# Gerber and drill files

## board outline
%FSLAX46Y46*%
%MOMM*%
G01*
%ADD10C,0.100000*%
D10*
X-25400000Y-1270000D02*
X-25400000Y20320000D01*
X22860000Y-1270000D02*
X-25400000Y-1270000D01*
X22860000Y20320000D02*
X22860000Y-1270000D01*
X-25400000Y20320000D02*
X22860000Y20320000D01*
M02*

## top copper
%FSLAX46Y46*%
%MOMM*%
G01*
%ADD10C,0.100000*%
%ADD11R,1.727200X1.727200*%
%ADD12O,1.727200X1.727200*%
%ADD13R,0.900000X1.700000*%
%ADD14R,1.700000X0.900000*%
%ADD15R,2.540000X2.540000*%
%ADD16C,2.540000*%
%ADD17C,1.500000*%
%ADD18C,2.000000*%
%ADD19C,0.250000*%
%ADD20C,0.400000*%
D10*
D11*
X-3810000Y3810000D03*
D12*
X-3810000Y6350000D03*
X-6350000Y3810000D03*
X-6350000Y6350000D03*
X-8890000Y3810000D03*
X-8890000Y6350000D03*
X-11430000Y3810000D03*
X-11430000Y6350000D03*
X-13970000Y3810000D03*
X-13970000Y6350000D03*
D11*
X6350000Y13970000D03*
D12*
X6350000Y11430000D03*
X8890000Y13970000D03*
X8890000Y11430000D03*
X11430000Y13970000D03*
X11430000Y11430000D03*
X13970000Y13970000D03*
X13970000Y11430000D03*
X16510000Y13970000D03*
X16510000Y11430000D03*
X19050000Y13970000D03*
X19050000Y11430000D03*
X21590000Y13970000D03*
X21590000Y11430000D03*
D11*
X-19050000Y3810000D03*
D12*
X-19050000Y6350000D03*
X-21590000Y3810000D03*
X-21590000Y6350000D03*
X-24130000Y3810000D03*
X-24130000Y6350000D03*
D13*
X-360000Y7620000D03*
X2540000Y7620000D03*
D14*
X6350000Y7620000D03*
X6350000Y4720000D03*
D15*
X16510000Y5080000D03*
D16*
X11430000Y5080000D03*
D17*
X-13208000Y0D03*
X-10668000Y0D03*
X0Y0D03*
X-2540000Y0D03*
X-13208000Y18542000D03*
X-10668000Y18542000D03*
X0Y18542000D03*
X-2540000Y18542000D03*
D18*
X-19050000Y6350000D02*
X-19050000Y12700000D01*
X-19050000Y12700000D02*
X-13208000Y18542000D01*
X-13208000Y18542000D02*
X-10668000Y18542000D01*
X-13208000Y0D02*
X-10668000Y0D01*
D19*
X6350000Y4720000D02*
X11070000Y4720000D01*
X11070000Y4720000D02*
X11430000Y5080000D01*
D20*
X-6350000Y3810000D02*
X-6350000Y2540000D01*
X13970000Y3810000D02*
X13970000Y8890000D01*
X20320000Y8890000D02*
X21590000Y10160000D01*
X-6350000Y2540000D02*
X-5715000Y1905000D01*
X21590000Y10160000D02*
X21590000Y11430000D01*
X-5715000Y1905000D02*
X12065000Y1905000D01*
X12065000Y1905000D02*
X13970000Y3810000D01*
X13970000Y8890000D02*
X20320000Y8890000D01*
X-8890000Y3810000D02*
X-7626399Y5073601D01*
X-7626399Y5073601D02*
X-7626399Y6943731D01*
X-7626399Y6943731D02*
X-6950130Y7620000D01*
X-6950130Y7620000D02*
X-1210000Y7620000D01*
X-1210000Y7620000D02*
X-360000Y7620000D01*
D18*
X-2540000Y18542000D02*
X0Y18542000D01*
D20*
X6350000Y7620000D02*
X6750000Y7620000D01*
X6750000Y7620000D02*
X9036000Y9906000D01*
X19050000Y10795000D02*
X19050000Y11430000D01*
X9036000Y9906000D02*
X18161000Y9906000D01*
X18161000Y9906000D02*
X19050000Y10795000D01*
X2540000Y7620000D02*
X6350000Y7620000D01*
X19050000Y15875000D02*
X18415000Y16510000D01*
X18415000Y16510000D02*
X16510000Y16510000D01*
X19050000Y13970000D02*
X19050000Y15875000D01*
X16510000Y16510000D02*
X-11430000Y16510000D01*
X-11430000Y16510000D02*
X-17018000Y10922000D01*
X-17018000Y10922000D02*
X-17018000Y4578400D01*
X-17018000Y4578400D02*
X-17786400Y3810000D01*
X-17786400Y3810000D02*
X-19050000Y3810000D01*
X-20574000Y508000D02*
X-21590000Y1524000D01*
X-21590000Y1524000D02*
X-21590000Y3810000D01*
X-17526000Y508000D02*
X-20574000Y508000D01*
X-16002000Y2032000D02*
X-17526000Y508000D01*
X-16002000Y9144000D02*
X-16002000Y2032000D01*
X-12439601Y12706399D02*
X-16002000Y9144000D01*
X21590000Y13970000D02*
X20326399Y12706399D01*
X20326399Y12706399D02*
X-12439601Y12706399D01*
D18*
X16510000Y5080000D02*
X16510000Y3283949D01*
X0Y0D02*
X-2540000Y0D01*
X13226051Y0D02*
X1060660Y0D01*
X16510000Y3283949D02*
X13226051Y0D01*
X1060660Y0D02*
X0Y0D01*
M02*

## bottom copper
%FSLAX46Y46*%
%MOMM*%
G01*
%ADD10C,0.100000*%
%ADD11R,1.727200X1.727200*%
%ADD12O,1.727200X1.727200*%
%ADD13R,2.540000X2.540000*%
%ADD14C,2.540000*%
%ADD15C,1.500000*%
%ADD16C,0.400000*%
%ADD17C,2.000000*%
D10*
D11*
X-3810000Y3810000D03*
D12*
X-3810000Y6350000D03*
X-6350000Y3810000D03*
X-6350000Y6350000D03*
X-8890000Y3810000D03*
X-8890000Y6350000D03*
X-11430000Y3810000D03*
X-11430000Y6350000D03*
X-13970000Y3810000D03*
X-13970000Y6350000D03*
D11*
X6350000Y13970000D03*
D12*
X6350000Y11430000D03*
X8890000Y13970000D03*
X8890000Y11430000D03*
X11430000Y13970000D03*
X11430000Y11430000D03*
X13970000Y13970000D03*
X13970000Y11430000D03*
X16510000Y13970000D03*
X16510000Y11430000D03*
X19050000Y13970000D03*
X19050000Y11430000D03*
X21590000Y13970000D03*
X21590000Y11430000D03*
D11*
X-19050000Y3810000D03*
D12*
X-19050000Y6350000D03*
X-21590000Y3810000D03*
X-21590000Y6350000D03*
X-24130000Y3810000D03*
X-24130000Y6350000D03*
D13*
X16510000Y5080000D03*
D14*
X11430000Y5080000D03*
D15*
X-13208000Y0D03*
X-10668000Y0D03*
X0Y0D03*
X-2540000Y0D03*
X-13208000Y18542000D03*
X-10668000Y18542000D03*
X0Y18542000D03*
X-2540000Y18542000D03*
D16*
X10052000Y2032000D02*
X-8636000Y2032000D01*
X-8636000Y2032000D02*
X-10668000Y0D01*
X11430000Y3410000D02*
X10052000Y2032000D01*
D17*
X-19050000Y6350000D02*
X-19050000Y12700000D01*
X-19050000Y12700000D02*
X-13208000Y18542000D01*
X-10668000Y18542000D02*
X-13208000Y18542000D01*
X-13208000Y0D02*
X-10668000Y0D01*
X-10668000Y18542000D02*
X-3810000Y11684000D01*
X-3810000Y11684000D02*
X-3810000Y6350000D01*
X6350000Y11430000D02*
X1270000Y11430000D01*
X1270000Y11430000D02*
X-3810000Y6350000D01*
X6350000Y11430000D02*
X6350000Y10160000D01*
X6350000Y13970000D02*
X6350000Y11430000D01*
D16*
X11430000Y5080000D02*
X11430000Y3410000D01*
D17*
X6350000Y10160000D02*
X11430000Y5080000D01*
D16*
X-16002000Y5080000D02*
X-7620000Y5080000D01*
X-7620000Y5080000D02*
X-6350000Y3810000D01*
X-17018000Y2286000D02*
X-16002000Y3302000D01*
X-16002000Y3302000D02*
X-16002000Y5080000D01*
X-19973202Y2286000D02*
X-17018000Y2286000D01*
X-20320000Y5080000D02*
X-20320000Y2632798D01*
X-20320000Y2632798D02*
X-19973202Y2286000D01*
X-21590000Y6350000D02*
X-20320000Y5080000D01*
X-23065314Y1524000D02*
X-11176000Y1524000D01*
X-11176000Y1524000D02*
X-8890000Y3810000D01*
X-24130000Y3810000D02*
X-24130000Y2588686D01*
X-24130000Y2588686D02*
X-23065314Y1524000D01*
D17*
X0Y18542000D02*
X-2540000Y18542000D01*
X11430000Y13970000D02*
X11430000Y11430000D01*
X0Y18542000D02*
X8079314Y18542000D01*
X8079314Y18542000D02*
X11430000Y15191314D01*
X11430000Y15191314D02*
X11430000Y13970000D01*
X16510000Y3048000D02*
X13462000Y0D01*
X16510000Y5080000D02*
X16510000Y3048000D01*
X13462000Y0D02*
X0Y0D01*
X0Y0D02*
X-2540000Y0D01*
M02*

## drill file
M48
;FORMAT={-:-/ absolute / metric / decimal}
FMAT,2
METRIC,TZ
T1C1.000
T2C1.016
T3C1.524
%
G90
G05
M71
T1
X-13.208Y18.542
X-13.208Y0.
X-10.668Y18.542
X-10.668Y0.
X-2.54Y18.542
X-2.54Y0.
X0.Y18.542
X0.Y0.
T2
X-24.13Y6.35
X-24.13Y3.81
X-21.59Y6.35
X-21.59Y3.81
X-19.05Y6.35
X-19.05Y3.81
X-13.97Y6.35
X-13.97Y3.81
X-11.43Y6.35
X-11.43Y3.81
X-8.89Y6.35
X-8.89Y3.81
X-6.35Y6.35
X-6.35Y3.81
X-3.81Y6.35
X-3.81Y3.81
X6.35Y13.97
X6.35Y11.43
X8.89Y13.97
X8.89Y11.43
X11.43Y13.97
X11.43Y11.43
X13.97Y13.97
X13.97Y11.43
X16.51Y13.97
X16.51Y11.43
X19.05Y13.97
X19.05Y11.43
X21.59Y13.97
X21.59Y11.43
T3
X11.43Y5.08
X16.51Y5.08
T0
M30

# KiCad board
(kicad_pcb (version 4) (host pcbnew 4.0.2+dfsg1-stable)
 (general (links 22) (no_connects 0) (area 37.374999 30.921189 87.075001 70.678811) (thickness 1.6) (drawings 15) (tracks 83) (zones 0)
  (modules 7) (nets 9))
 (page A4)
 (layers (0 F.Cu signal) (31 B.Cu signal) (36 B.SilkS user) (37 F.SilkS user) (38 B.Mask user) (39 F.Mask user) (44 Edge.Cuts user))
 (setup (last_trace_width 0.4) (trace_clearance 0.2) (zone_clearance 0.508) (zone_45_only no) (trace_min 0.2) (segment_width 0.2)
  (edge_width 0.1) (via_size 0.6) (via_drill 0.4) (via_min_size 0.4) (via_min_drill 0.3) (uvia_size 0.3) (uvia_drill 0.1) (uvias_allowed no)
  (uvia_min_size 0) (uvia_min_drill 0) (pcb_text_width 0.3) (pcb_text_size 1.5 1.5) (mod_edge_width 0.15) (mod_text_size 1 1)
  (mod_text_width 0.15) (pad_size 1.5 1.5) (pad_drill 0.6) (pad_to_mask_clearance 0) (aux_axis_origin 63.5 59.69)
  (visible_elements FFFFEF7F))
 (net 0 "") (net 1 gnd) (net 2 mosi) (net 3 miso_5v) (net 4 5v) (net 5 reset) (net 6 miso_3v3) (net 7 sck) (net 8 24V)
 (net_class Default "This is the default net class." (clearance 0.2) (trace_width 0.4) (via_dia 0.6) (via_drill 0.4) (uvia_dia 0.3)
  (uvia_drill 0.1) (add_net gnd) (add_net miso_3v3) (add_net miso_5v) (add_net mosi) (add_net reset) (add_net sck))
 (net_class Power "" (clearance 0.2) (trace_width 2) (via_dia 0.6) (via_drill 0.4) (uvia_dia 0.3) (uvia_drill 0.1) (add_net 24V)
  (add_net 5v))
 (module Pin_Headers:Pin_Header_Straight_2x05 (layer B.Cu) (at 59.69 55.88 90)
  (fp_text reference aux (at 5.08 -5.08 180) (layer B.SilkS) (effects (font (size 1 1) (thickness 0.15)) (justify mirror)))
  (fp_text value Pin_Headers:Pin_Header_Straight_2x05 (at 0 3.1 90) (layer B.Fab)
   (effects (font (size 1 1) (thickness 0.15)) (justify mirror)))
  (pad 1 thru_hole rect (at 0 0 90) (size 1.7272 1.7272) (drill 1.016) (layers *.Cu *.Mask B.SilkS))
  (pad 2 thru_hole oval (at 2.54 0 90) (size 1.7272 1.7272) (drill 1.016) (layers *.Cu *.Mask B.SilkS) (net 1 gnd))
  (pad 3 thru_hole oval (at 0 -2.54 90) (size 1.7272 1.7272) (drill 1.016) (layers *.Cu *.Mask B.SilkS) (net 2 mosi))
  (pad 4 thru_hole oval (at 2.54 -2.54 90) (size 1.7272 1.7272) (drill 1.016) (layers *.Cu *.Mask B.SilkS))
  (pad 5 thru_hole oval (at 0 -5.08 90) (size 1.7272 1.7272) (drill 1.016) (layers *.Cu *.Mask B.SilkS) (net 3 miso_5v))
  (pad 6 thru_hole oval (at 2.54 -5.08 90) (size 1.7272 1.7272) (drill 1.016) (layers *.Cu *.Mask B.SilkS))
  (pad 7 thru_hole oval (at 0 -7.62 90) (size 1.7272 1.7272) (drill 1.016) (layers *.Cu *.Mask B.SilkS))
  (pad 8 thru_hole oval (at 2.54 -7.62 90) (size 1.7272 1.7272) (drill 1.016) (layers *.Cu *.Mask B.SilkS))
  (pad 9 thru_hole oval (at 0 -10.16 90) (size 1.7272 1.7272) (drill 1.016) (layers *.Cu *.Mask B.SilkS))
  (pad 10 thru_hole oval (at 2.54 -10.16 90) (size 1.7272 1.7272) (drill 1.016) (layers *.Cu *.Mask B.SilkS)))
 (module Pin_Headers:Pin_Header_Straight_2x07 (layer B.Cu) (at 69.85 45.72 270)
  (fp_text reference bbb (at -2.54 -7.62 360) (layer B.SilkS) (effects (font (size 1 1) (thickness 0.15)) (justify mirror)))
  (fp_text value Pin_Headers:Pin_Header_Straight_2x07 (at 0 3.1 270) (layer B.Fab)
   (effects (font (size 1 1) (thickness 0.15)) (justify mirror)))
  (pad 1 thru_hole rect (at 0 0 270) (size 1.7272 1.7272) (drill 1.016) (layers *.Cu *.Mask B.SilkS) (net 1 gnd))
  (pad 2 thru_hole oval (at 2.54 0 270) (size 1.7272 1.7272) (drill 1.016) (layers *.Cu *.Mask B.SilkS) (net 1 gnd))
  (pad 3 thru_hole oval (at 0 -2.54 270) (size 1.7272 1.7272) (drill 1.016) (layers *.Cu *.Mask B.SilkS))
  (pad 4 thru_hole oval (at 2.54 -2.54 270) (size 1.7272 1.7272) (drill 1.016) (layers *.Cu *.Mask B.SilkS))
  (pad 5 thru_hole oval (at 0 -5.08 270) (size 1.7272 1.7272) (drill 1.016) (layers *.Cu *.Mask B.SilkS) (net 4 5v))
  (pad 6 thru_hole oval (at 2.54 -5.08 270) (size 1.7272 1.7272) (drill 1.016) (layers *.Cu *.Mask B.SilkS) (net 4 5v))
  (pad 7 thru_hole oval (at 0 -7.62 270) (size 1.7272 1.7272) (drill 1.016) (layers *.Cu *.Mask B.SilkS))
  (pad 8 thru_hole oval (at 2.54 -7.62 270) (size 1.7272 1.7272) (drill 1.016) (layers *.Cu *.Mask B.SilkS))
  (pad 9 thru_hole oval (at 0 -10.16 270) (size 1.7272 1.7272) (drill 1.016) (layers *.Cu *.Mask B.SilkS))
  (pad 10 thru_hole oval (at 2.54 -10.16 270) (size 1.7272 1.7272) (drill 1.016) (layers *.Cu *.Mask B.SilkS))
  (pad 11 thru_hole oval (at 0 -12.7 270) (size 1.7272 1.7272) (drill 1.016) (layers *.Cu *.Mask B.SilkS) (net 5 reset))
  (pad 12 thru_hole oval (at 2.54 -12.7 270) (size 1.7272 1.7272) (drill 1.016) (layers *.Cu *.Mask B.SilkS) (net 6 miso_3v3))
  (pad 13 thru_hole oval (at 0 -15.24 270) (size 1.7272 1.7272) (drill 1.016) (layers *.Cu *.Mask B.SilkS) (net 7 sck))
  (pad 14 thru_hole oval (at 2.54 -15.24 270) (size 1.7272 1.7272) (drill 1.016) (layers *.Cu *.Mask B.SilkS) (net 2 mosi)))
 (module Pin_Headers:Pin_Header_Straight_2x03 (layer B.Cu) (at 44.45 55.88 90)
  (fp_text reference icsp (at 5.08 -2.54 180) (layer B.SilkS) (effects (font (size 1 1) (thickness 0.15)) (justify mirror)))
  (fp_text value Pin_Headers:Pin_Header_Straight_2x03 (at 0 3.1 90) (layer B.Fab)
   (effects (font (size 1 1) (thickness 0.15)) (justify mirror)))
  (pad 1 thru_hole rect (at 0 0 90) (size 1.7272 1.7272) (drill 1.016) (layers *.Cu *.Mask B.SilkS) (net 5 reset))
  (pad 2 thru_hole oval (at 2.54 0 90) (size 1.7272 1.7272) (drill 1.016) (layers *.Cu *.Mask B.SilkS) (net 1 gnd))
  (pad 3 thru_hole oval (at 0 -2.54 90) (size 1.7272 1.7272) (drill 1.016) (layers *.Cu *.Mask B.SilkS) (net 7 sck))
  (pad 4 thru_hole oval (at 2.54 -2.54 90) (size 1.7272 1.7272) (drill 1.016) (layers *.Cu *.Mask B.SilkS) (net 2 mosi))
  (pad 5 thru_hole oval (at 0 -5.08 90) (size 1.7272 1.7272) (drill 1.016) (layers *.Cu *.Mask B.SilkS) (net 3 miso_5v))
  (pad 6 thru_hole oval (at 2.54 -5.08 90) (size 1.7272 1.7272) (drill 1.016) (layers *.Cu *.Mask B.SilkS)))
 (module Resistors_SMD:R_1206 (layer F.Cu) (at 64.59 52.07)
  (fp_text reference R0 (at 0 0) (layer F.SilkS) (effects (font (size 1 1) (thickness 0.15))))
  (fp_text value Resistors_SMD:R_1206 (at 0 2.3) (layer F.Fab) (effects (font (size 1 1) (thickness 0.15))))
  (pad 1 smd rect (at -1.45 0) (size 0.9 1.7) (layers F.Cu F.Mask) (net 3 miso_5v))
  (pad 2 smd rect (at 1.45 0) (size 0.9 1.7) (layers F.Cu F.Mask) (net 6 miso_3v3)))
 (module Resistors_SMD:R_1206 (layer F.Cu) (at 69.85 53.52 270)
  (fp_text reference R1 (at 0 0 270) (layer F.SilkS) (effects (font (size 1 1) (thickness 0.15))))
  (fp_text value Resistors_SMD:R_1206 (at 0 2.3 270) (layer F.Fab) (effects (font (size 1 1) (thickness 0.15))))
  (pad 1 smd rect (at -1.45 0 270) (size 0.9 1.7) (layers F.Cu F.Mask) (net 6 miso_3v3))
  (pad 2 smd rect (at 1.45 0 270) (size 0.9 1.7) (layers F.Cu F.Mask) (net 1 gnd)))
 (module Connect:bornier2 (layer F.Cu) (at 77.47 54.61 180)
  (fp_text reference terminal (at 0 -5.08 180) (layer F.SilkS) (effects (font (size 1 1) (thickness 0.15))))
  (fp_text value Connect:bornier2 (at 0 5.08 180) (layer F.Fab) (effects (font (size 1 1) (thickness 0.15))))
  (pad 1 thru_hole rect (at -2.54 0 180) (size 2.54 2.54) (drill 1.524) (layers *.Cu *.Mask F.SilkS) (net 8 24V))
  (pad 2 thru_hole circle (at 2.54 0 180) (size 2.54 2.54) (drill 1.524) (layers *.Cu *.Mask F.SilkS) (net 1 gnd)))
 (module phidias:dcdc (layer F.Cu) (at 63.5 59.69 90)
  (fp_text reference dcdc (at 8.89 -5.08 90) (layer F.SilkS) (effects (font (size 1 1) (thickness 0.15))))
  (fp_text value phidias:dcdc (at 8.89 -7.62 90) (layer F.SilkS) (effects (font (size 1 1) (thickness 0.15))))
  (pad gnd thru_hole circle (at 0 -13.208 90) (size 1.5 1.5) (drill 1) (layers *.Cu *.Mask F.SilkS) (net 1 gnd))
  (pad gnd thru_hole circle (at 0 -10.668 90) (size 1.5 1.5) (drill 1) (layers *.Cu *.Mask F.SilkS) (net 1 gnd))
  (pad in thru_hole circle (at 0 0 90) (size 1.5 1.5) (drill 1) (layers *.Cu *.Mask F.SilkS) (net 8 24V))
  (pad in thru_hole circle (at 0 -2.54 90) (size 1.5 1.5) (drill 1) (layers *.Cu *.Mask F.SilkS) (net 8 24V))
  (pad gnd thru_hole circle (at 18.542 -13.208 90) (size 1.5 1.5) (drill 1) (layers *.Cu *.Mask F.SilkS) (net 1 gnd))
  (pad gnd thru_hole circle (at 18.542 -10.668 90) (size 1.5 1.5) (drill 1) (layers *.Cu *.Mask F.SilkS) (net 1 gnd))
  (pad out thru_hole circle (at 18.542 0 90) (size 1.5 1.5) (drill 1) (layers *.Cu *.Mask F.SilkS) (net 4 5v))
  (pad out thru_hole circle (at 18.542 -2.54 90) (size 1.5 1.5) (drill 1) (layers *.Cu *.Mask F.SilkS) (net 4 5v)))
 (gr_line (start 38.1 60.96) (end 38.1 39.37) (layer Edge.Cuts) (width 0.1))
 (gr_line (start 86.36 60.96) (end 38.1 60.96) (layer Edge.Cuts) (width 0.1))
 (gr_line (start 86.36 39.37) (end 86.36 60.96) (layer Edge.Cuts) (width 0.1))
 (gr_line (start 38.1 39.37) (end 86.36 39.37) (layer Edge.Cuts) (width 0.1))
 (segment (start 73.552 57.658) (end 54.864 57.658) (width 0.4) (layer B.Cu) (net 1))
 (segment (start 54.864 57.658) (end 52.832 59.69) (width 0.4) (layer B.Cu) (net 1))
 (segment (start 74.93 56.28) (end 73.552 57.658) (width 0.4) (layer B.Cu) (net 1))
 (segment (start 44.45 53.34) (end 44.45 46.99) (width 2) (layer B.Cu) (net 1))
 (segment (start 44.45 46.99) (end 50.292 41.148) (width 2) (layer B.Cu) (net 1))
 (segment (start 52.832 41.148) (end 50.292 41.148) (width 2) (layer B.Cu) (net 1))
 (segment (start 50.292 59.69) (end 52.832 59.69) (width 2) (layer B.Cu) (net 1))
 (segment (start 44.45 53.34) (end 44.45 46.99) (width 2) (layer F.Cu) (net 1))
 (segment (start 44.45 46.99) (end 50.292 41.148) (width 2) (layer F.Cu) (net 1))
 (segment (start 50.292 41.148) (end 52.832 41.148) (width 2) (layer F.Cu) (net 1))
 (segment (start 50.292 59.69) (end 52.832 59.69) (width 2) (layer F.Cu) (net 1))
 (segment (start 52.832 41.148) (end 59.69 48.006) (width 2) (layer B.Cu) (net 1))
 (segment (start 59.69 48.006) (end 59.69 53.34) (width 2) (layer B.Cu) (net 1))
 (segment (start 69.85 48.26) (end 64.77 48.26) (width 2) (layer B.Cu) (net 1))
 (segment (start 64.77 48.26) (end 59.69 53.34) (width 2) (layer B.Cu) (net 1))
 (segment (start 69.85 48.26) (end 69.85 49.53) (width 2) (layer B.Cu) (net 1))
 (segment (start 69.85 45.72) (end 69.85 48.26) (width 2) (layer B.Cu) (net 1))
 (segment (start 69.85 54.97) (end 74.57 54.97) (width 0.25) (layer F.Cu) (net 1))
 (segment (start 74.93 54.61) (end 74.93 56.28) (width 0.4) (layer B.Cu) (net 1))
 (segment (start 69.85 49.53) (end 74.93 54.61) (width 2) (layer B.Cu) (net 1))
 (segment (start 74.57 54.97) (end 74.93 54.61) (width 0.25) (layer F.Cu) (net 1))
 (segment (start 57.15 55.88) (end 57.15 57.15) (width 0.4) (layer F.Cu) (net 2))
 (segment (start 77.47 55.88) (end 77.47 50.8) (width 0.4) (layer F.Cu) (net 2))
 (segment (start 83.82 50.8) (end 85.09 49.53) (width 0.4) (layer F.Cu) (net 2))
 (segment (start 57.15 57.15) (end 57.785 57.785) (width 0.4) (layer F.Cu) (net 2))
 (segment (start 85.09 49.53) (end 85.09 48.26) (width 0.4) (layer F.Cu) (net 2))
 (segment (start 57.785 57.785) (end 75.565 57.785) (width 0.4) (layer F.Cu) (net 2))
 (segment (start 75.565 57.785) (end 77.47 55.88) (width 0.4) (layer F.Cu) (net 2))
 (segment (start 77.47 50.8) (end 83.82 50.8) (width 0.4) (layer F.Cu) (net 2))
 (segment (start 47.498 54.61) (end 55.88 54.61) (width 0.4) (layer B.Cu) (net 2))
 (segment (start 55.88 54.61) (end 57.15 55.88) (width 0.4) (layer B.Cu) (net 2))
 (segment (start 46.482 57.404) (end 47.498 56.388) (width 0.4) (layer B.Cu) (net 2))
 (segment (start 47.498 56.388) (end 47.498 54.61) (width 0.4) (layer B.Cu) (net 2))
 (segment (start 43.526798 57.404) (end 46.482 57.404) (width 0.4) (layer B.Cu) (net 2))
 (segment (start 43.18 54.61) (end 43.18 57.057202) (width 0.4) (layer B.Cu) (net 2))
 (segment (start 43.18 57.057202) (end 43.526798 57.404) (width 0.4) (layer B.Cu) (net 2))
 (segment (start 41.91 53.34) (end 43.18 54.61) (width 0.4) (layer B.Cu) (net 2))
 (segment (start 40.434686 58.166) (end 52.324 58.166) (width 0.4) (layer B.Cu) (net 3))
 (segment (start 52.324 58.166) (end 54.61 55.88) (width 0.4) (layer B.Cu) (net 3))
 (segment (start 39.37 55.88) (end 39.37 57.101314) (width 0.4) (layer B.Cu) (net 3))
 (segment (start 39.37 57.101314) (end 40.434686 58.166) (width 0.4) (layer B.Cu) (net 3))
 (segment (start 54.61 55.88) (end 55.873601 54.616399) (width 0.4) (layer F.Cu) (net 3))
 (segment (start 55.873601 54.616399) (end 55.873601 52.746269) (width 0.4) (layer F.Cu) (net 3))
 (segment (start 55.873601 52.746269) (end 56.54987 52.07) (width 0.4) (layer F.Cu) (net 3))
 (segment (start 56.54987 52.07) (end 62.29 52.07) (width 0.4) (layer F.Cu) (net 3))
 (segment (start 62.29 52.07) (end 63.14 52.07) (width 0.4) (layer F.Cu) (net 3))
 (segment (start 60.96 41.148) (end 63.5 41.148) (width 2) (layer F.Cu) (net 4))
 (segment (start 63.5 41.148) (end 60.96 41.148) (width 2) (layer B.Cu) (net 4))
 (segment (start 74.93 45.72) (end 74.93 48.26) (width 2) (layer B.Cu) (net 4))
 (segment (start 63.5 41.148) (end 71.579314 41.148) (width 2) (layer B.Cu) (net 4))
 (segment (start 71.579314 41.148) (end 74.93 44.498686) (width 2) (layer B.Cu) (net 4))
 (segment (start 74.93 44.498686) (end 74.93 45.72) (width 2) (layer B.Cu) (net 4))
 (segment (start 69.85 52.07) (end 70.25 52.07) (width 0.4) (layer F.Cu) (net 6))
 (segment (start 70.25 52.07) (end 72.536 49.784) (width 0.4) (layer F.Cu) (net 6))
 (segment (start 82.55 48.895) (end 82.55 48.26) (width 0.4) (layer F.Cu) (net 6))
 (segment (start 72.536 49.784) (end 81.661 49.784) (width 0.4) (layer F.Cu) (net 6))
 (segment (start 81.661 49.784) (end 82.55 48.895) (width 0.4) (layer F.Cu) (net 6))
 (segment (start 66.04 52.07) (end 69.85 52.07) (width 0.4) (layer F.Cu) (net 6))
 (segment (start 82.55 43.815) (end 81.915 43.18) (width 0.4) (layer F.Cu) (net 5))
 (segment (start 81.915 43.18) (end 80.01 43.18) (width 0.4) (layer F.Cu) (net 5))
 (segment (start 82.55 45.72) (end 82.55 43.815) (width 0.4) (layer F.Cu) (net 5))
 (segment (start 80.01 43.18) (end 52.07 43.18) (width 0.4) (layer F.Cu) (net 5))
 (segment (start 52.07 43.18) (end 46.482 48.768) (width 0.4) (layer F.Cu) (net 5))
 (segment (start 46.482 48.768) (end 46.482 55.1116) (width 0.4) (layer F.Cu) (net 5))
 (segment (start 46.482 55.1116) (end 45.7136 55.88) (width 0.4) (layer F.Cu) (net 5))
 (segment (start 45.7136 55.88) (end 44.45 55.88) (width 0.4) (layer F.Cu) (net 5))
 (segment (start 42.926 59.182) (end 41.91 58.166) (width 0.4) (layer F.Cu) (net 7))
 (segment (start 41.91 58.166) (end 41.91 55.88) (width 0.4) (layer F.Cu) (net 7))
 (segment (start 45.974 59.182) (end 42.926 59.182) (width 0.4) (layer F.Cu) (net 7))
 (segment (start 47.498 57.658) (end 45.974 59.182) (width 0.4) (layer F.Cu) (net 7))
 (segment (start 47.498 50.546) (end 47.498 57.658) (width 0.4) (layer F.Cu) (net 7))
 (segment (start 51.060399 46.983601) (end 47.498 50.546) (width 0.4) (layer F.Cu) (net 7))
 (segment (start 85.09 45.72) (end 83.826399 46.983601) (width 0.4) (layer F.Cu) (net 7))
 (segment (start 83.826399 46.983601) (end 51.060399 46.983601) (width 0.4) (layer F.Cu) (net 7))
 (segment (start 80.01 56.642) (end 76.962 59.69) (width 2) (layer B.Cu) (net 8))
 (segment (start 80.01 54.61) (end 80.01 56.642) (width 2) (layer B.Cu) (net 8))
 (segment (start 80.01 54.61) (end 80.01 56.406051) (width 2) (layer F.Cu) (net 8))
 (segment (start 63.5 59.69) (end 60.96 59.69) (width 2) (layer F.Cu) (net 8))
 (segment (start 76.962 59.69) (end 63.5 59.69) (width 2) (layer B.Cu) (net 8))
 (segment (start 76.726051 59.69) (end 64.56066 59.69) (width 2) (layer F.Cu) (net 8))
 (segment (start 80.01 56.406051) (end 76.726051 59.69) (width 2) (layer F.Cu) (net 8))
 (segment (start 64.56066 59.69) (end 63.5 59.69) (width 2) (layer F.Cu) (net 8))
 (segment (start 63.5 59.69) (end 60.96 59.69) (width 2) (layer B.Cu) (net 8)))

